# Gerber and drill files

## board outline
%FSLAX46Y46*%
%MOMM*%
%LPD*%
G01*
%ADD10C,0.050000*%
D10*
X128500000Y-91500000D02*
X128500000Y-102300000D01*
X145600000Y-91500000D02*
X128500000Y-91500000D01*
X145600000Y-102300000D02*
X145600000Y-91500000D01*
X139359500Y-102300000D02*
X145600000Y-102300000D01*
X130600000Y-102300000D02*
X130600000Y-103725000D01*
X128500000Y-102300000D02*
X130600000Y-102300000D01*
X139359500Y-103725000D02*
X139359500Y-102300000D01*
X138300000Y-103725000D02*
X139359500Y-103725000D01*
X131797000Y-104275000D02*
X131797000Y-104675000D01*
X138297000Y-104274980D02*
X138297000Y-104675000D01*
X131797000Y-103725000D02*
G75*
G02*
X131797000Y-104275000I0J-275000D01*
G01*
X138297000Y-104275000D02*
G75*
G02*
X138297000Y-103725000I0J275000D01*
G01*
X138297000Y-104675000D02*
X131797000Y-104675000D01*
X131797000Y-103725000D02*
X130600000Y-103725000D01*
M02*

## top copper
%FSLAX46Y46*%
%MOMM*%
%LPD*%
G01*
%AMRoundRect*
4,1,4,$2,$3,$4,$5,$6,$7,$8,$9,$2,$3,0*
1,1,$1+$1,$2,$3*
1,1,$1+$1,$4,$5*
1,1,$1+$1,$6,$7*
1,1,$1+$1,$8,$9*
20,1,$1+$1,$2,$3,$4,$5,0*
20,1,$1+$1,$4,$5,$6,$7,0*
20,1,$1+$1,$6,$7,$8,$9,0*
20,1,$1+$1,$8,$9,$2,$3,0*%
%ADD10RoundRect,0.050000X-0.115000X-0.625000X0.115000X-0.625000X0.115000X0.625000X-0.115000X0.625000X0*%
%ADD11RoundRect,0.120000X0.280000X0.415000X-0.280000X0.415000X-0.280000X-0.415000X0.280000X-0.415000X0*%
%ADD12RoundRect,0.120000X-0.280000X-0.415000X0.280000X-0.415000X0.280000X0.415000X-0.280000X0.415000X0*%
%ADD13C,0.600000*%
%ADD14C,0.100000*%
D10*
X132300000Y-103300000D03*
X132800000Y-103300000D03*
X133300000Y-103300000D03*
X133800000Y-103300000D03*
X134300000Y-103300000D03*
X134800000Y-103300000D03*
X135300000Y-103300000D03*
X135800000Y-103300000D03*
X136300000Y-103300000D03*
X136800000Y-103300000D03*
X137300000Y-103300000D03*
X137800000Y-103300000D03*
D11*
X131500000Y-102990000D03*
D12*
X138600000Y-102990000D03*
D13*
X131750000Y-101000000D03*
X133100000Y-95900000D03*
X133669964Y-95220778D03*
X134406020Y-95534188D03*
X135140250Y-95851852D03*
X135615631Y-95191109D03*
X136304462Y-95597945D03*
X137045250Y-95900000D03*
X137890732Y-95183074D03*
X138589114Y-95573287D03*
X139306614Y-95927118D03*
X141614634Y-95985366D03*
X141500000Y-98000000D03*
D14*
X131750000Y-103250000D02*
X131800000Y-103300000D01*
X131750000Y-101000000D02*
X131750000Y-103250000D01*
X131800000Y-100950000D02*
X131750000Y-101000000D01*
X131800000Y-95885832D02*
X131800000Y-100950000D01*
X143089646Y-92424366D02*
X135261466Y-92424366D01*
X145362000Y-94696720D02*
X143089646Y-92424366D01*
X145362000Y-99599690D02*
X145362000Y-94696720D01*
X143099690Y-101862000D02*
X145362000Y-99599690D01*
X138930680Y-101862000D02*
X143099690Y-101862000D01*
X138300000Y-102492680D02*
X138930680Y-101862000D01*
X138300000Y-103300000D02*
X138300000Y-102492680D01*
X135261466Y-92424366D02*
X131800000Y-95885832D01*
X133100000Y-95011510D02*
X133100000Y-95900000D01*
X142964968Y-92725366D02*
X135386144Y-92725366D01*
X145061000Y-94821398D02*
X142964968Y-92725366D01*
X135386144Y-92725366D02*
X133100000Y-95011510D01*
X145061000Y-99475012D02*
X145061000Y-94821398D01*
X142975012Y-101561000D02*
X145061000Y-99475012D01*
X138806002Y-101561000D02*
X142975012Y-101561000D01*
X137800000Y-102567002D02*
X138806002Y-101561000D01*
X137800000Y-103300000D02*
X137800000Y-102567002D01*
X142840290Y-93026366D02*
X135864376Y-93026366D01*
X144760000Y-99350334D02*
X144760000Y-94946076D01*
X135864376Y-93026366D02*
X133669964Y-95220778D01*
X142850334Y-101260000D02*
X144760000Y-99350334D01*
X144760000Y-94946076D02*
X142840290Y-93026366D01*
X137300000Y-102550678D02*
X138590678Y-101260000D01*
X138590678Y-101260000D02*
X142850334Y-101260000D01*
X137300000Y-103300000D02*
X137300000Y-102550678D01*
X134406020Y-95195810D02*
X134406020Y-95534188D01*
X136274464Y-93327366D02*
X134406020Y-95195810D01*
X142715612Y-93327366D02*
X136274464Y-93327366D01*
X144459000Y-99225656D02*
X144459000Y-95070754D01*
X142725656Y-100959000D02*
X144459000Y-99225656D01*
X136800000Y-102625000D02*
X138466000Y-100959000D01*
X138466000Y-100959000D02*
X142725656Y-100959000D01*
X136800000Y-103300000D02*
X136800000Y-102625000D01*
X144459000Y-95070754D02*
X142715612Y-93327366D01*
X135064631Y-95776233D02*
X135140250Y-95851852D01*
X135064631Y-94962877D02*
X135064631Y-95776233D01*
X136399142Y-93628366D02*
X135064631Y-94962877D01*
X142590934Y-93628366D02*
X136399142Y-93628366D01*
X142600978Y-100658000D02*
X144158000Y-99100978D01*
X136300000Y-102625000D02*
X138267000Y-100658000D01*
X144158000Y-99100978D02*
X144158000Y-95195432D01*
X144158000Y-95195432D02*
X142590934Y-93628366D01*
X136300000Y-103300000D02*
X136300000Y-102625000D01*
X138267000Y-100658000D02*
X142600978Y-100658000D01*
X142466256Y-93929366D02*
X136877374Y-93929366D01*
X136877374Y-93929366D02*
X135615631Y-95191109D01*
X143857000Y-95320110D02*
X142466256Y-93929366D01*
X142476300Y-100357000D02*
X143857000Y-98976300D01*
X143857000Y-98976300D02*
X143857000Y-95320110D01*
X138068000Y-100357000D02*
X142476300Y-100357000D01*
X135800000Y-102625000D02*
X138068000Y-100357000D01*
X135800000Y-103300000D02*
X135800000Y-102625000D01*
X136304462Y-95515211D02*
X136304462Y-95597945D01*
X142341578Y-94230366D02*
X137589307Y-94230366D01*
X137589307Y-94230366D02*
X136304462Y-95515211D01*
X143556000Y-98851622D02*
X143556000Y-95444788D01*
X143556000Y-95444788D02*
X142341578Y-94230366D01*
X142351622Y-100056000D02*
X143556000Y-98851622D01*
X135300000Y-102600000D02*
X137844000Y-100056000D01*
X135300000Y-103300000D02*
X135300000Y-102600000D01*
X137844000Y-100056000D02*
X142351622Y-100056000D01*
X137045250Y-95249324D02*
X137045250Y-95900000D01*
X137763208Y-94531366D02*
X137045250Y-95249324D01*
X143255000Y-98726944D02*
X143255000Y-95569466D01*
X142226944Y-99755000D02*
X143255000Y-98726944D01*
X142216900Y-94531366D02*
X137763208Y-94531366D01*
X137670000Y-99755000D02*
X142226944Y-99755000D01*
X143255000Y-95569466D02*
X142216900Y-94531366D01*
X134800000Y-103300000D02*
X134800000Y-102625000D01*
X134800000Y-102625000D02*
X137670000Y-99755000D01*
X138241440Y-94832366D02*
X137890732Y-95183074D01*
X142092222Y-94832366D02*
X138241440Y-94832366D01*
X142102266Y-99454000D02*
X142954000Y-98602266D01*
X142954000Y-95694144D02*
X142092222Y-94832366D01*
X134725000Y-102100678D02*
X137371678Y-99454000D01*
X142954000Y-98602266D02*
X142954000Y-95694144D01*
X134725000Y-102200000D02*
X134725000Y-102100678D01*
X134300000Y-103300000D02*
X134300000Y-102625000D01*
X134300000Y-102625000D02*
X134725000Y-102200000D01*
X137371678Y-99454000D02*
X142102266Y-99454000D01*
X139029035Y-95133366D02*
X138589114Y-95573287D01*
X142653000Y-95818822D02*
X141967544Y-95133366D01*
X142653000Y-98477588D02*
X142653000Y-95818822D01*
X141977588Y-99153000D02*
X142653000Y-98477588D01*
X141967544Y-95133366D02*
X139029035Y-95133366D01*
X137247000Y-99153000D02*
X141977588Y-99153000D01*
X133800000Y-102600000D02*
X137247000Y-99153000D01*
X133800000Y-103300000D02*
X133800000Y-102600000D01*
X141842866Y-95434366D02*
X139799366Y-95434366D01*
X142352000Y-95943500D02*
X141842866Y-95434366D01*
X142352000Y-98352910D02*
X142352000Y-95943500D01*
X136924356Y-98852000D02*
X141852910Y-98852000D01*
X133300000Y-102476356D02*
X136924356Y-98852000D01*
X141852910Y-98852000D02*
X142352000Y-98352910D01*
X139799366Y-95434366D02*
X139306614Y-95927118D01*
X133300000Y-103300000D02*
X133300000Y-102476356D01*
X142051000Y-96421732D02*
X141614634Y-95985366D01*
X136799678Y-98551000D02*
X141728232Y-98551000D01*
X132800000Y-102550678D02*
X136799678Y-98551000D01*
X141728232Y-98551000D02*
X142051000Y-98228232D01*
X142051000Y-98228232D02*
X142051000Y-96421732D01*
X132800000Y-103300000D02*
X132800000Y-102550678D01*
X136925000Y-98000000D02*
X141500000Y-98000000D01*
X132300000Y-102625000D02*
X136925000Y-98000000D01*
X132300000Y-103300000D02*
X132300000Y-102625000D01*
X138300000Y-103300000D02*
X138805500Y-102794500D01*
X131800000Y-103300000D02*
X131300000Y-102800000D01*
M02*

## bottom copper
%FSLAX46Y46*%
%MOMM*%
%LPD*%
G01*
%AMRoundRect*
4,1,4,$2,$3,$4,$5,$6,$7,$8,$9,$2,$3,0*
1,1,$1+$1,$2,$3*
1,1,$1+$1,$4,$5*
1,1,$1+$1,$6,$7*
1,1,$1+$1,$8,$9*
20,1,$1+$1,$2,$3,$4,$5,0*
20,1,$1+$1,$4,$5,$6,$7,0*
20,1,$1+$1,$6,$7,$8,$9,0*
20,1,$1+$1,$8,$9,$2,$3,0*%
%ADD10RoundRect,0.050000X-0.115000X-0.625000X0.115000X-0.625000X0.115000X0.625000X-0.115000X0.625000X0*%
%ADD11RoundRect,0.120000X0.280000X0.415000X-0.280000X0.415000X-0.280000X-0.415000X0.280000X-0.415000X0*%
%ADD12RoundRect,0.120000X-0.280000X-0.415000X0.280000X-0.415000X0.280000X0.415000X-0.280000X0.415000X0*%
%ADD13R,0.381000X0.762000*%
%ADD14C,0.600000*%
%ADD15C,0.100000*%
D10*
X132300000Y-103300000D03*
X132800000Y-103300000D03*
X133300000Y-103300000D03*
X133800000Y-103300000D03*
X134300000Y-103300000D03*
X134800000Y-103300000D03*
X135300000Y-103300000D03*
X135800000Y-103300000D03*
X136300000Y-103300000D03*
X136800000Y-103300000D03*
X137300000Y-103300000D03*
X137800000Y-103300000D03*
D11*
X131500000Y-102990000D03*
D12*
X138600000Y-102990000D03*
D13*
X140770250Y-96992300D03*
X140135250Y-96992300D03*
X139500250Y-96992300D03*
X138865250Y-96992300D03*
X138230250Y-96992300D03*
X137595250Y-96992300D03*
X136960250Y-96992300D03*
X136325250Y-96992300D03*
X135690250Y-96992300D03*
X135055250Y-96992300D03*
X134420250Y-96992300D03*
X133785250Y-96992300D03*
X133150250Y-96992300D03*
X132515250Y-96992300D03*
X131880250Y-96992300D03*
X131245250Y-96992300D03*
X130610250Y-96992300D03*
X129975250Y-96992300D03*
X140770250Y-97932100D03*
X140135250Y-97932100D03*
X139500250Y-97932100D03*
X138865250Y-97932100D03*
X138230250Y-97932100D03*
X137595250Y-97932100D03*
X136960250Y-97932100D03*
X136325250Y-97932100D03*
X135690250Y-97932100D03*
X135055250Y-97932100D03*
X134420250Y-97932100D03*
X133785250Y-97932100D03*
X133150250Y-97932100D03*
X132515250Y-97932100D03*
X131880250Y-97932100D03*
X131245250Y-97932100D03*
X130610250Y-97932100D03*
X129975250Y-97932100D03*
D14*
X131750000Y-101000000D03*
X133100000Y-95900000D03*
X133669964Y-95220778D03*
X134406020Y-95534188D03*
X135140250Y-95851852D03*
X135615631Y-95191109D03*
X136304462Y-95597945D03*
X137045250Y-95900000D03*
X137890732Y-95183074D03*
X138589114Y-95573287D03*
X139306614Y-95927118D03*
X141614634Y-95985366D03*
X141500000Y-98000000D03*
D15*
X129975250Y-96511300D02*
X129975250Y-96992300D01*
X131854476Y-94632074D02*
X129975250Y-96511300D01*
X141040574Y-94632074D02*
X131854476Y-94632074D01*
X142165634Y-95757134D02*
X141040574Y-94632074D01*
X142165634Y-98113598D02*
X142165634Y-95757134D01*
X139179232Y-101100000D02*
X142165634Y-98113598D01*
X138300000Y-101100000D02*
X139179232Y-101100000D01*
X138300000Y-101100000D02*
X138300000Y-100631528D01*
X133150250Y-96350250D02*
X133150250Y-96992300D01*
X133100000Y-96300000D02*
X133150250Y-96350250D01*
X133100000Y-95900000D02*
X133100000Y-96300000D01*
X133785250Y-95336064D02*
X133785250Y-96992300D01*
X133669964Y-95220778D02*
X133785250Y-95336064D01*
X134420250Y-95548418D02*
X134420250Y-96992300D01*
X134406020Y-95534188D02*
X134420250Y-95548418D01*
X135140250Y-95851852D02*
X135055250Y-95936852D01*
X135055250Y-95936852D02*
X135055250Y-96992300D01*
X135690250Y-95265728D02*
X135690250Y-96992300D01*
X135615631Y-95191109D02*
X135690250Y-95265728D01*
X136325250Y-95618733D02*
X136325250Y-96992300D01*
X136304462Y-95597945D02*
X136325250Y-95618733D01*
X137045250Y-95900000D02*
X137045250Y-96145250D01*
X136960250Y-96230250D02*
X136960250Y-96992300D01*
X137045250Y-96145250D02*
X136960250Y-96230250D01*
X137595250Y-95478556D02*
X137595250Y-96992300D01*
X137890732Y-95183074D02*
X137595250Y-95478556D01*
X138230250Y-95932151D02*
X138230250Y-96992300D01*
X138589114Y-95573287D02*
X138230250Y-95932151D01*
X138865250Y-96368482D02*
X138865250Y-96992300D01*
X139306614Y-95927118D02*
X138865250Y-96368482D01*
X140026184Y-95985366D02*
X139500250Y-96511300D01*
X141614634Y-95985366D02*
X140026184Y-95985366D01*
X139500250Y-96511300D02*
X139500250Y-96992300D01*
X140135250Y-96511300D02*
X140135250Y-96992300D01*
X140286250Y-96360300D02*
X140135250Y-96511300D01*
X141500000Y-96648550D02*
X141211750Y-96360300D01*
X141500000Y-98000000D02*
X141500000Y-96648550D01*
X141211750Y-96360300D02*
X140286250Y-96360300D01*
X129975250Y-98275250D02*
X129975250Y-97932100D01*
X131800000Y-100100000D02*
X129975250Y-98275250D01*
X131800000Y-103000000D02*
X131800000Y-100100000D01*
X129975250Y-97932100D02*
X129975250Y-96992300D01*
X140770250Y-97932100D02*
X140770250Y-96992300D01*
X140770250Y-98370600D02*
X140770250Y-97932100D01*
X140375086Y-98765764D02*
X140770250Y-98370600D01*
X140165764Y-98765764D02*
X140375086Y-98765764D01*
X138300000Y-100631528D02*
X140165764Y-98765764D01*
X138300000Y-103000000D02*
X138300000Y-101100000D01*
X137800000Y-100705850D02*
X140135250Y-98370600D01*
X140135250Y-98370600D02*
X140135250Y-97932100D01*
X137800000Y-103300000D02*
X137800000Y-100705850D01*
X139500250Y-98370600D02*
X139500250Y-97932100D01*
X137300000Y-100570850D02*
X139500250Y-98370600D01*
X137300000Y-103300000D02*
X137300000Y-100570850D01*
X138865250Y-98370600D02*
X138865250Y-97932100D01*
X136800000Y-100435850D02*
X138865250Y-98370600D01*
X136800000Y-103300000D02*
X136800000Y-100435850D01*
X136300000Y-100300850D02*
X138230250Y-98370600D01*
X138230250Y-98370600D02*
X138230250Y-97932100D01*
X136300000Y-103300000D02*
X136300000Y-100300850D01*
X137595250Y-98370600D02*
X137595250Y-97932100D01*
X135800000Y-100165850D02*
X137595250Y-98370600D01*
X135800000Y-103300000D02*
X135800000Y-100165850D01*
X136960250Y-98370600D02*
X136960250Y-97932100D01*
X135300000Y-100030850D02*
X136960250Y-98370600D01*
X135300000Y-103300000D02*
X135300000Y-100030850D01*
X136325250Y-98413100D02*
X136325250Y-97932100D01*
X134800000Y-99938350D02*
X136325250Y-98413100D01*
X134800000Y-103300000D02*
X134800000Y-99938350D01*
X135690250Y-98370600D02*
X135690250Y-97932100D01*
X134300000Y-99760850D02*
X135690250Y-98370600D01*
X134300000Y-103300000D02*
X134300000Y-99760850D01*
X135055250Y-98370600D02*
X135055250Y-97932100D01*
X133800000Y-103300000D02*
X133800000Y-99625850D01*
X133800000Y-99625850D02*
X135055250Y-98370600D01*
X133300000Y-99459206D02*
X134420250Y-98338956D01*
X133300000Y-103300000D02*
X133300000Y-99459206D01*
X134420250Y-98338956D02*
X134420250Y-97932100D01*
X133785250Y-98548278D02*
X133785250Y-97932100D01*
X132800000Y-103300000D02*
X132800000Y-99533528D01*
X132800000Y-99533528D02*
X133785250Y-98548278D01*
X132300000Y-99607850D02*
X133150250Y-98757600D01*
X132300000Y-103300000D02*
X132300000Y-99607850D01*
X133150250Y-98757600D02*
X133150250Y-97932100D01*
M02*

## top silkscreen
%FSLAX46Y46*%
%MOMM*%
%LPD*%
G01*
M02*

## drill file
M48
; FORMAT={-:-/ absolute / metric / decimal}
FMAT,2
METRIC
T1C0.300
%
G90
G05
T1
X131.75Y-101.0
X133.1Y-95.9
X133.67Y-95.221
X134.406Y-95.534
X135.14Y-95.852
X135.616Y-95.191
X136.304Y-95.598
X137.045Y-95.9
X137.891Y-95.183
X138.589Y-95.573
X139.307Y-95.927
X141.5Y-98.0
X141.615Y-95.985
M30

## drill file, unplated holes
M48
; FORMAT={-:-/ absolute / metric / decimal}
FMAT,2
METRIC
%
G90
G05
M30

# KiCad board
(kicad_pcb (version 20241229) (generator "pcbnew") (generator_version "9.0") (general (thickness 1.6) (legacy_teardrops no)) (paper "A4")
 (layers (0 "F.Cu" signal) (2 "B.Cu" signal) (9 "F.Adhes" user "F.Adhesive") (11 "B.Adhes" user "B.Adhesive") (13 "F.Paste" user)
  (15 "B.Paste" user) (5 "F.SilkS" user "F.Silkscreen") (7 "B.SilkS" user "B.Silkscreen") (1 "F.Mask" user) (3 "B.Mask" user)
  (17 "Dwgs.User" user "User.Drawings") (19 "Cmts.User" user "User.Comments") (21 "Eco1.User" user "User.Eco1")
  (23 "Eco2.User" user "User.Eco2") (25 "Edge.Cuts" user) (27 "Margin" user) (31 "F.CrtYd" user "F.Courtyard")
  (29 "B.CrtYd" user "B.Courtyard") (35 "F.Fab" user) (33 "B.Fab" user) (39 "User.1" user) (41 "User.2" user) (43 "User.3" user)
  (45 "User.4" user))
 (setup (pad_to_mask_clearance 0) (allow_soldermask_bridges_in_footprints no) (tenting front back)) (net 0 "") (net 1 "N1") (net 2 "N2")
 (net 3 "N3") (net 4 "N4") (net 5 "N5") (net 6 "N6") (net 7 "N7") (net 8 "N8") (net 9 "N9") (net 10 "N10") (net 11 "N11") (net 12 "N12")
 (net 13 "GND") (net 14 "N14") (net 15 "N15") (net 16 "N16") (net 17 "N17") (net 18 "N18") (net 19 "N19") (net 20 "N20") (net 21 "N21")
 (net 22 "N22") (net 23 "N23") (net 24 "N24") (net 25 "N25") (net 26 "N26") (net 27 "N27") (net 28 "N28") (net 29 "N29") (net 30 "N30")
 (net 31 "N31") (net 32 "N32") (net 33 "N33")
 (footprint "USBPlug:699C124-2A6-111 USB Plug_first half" (layer "F.Cu") (at 134.8 100.3)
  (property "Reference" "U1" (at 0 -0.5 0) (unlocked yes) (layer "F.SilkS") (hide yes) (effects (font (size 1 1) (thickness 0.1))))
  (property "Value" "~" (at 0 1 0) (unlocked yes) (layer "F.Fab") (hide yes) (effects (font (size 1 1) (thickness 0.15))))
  (pad "0" smd roundrect (at -2.5 3) (size 0.33 1.35) (layers "F.Cu" "F.Mask" "F.Paste") (roundrect_rratio 0.1515151515) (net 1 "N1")
   (thermal_bridge_angle 45))
  (pad "1" smd roundrect (at -2 3) (size 0.33 1.35) (layers "F.Cu" "F.Mask" "F.Paste") (roundrect_rratio 0.1515151515) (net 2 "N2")
   (thermal_bridge_angle 45))
  (pad "2" smd roundrect (at -1.5 3) (size 0.33 1.35) (layers "F.Cu" "F.Mask" "F.Paste") (roundrect_rratio 0.1515151515) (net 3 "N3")
   (thermal_bridge_angle 45))
  (pad "3" smd roundrect (at -1 3) (size 0.33 1.35) (layers "F.Cu" "F.Mask" "F.Paste") (roundrect_rratio 0.1515151515) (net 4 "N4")
   (thermal_bridge_angle 45))
  (pad "4" smd roundrect (at -0.5 3) (size 0.33 1.35) (layers "F.Cu" "F.Mask" "F.Paste") (roundrect_rratio 0.1515151515) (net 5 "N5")
   (thermal_bridge_angle 45))
  (pad "5" smd roundrect (at 0 3) (size 0.33 1.35) (layers "F.Cu" "F.Mask" "F.Paste") (roundrect_rratio 0.1515151515) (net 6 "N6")
   (thermal_bridge_angle 45))
  (pad "6" smd roundrect (at 0.5 3) (size 0.33 1.35) (layers "F.Cu" "F.Mask" "F.Paste") (roundrect_rratio 0.1515151515) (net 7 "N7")
   (thermal_bridge_angle 45))
  (pad "7" smd roundrect (at 1 3) (size 0.33 1.35) (layers "F.Cu" "F.Mask" "F.Paste") (roundrect_rratio 0.1515151515) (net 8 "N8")
   (thermal_bridge_angle 45))
  (pad "8" smd roundrect (at 1.5 3) (size 0.33 1.35) (layers "F.Cu" "F.Mask" "F.Paste") (roundrect_rratio 0.1515151515) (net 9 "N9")
   (thermal_bridge_angle 45))
  (pad "9" smd roundrect (at 2 3) (size 0.33 1.35) (layers "F.Cu" "F.Mask" "F.Paste") (roundrect_rratio 0.1515151515) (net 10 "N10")
   (thermal_bridge_angle 45))
  (pad "10" smd roundrect (at 2.5 3) (size 0.33 1.35) (layers "F.Cu" "F.Mask" "F.Paste") (roundrect_rratio 0.1515151515) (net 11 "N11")
   (thermal_bridge_angle 45))
  (pad "11" smd roundrect (at 3 3) (size 0.33 1.35) (layers "F.Cu" "F.Mask" "F.Paste") (roundrect_rratio 0.1515151515) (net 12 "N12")
   (thermal_bridge_angle 45))
  (pad "24" smd roundrect (at -3 3 180) (size 0.8 1.07) (drill (offset 0.3 0.31)) (layers "F.Cu" "F.Mask" "F.Paste") (roundrect_rratio 0.15)
   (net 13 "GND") (thermal_bridge_angle 45))
  (pad "25" smd roundrect (at 3.5 3) (size 0.8 1.07) (drill (offset 0.3 -0.31)) (layers "F.Cu" "F.Mask" "F.Paste") (roundrect_rratio 0.15)
   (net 13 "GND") (thermal_bridge_angle 45)))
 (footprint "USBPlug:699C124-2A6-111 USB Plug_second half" (layer "B.Cu") (at 134.8 106.3)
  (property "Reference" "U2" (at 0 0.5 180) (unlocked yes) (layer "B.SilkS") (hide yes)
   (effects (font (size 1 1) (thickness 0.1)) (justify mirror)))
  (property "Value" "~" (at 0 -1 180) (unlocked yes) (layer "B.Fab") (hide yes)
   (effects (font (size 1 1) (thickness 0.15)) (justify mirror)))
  (pad "12" smd roundrect (at -2.5 -3) (size 0.33 1.35) (layers "B.Cu" "B.Mask" "B.Paste") (roundrect_rratio 0.1515151515) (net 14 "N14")
   (thermal_bridge_angle 45))
  (pad "13" smd roundrect (at -2 -3) (size 0.33 1.35) (layers "B.Cu" "B.Mask" "B.Paste") (roundrect_rratio 0.1515151515) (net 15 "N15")
   (thermal_bridge_angle 45))
  (pad "14" smd roundrect (at -1.5 -3) (size 0.33 1.35) (layers "B.Cu" "B.Mask" "B.Paste") (roundrect_rratio 0.1515151515) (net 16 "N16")
   (thermal_bridge_angle 45))
  (pad "15" smd roundrect (at -1 -3) (size 0.33 1.35) (layers "B.Cu" "B.Mask" "B.Paste") (roundrect_rratio 0.1515151515) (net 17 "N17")
   (thermal_bridge_angle 45))
  (pad "16" smd roundrect (at -0.5 -3) (size 0.33 1.35) (layers "B.Cu" "B.Mask" "B.Paste") (roundrect_rratio 0.1515151515) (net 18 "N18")
   (thermal_bridge_angle 45))
  (pad "17" smd roundrect (at 0 -3) (size 0.33 1.35) (layers "B.Cu" "B.Mask" "B.Paste") (roundrect_rratio 0.1515151515) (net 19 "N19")
   (thermal_bridge_angle 45))
  (pad "18" smd roundrect (at 0.5 -3) (size 0.33 1.35) (layers "B.Cu" "B.Mask" "B.Paste") (roundrect_rratio 0.1515151515) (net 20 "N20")
   (thermal_bridge_angle 45))
  (pad "19" smd roundrect (at 1 -3) (size 0.33 1.35) (layers "B.Cu" "B.Mask" "B.Paste") (roundrect_rratio 0.1515151515) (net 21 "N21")
   (thermal_bridge_angle 45))
  (pad "20" smd roundrect (at 1.5 -3) (size 0.33 1.35) (layers "B.Cu" "B.Mask" "B.Paste") (roundrect_rratio 0.1515151515) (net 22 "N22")
   (thermal_bridge_angle 45))
  (pad "21" smd roundrect (at 2 -3) (size 0.33 1.35) (layers "B.Cu" "B.Mask" "B.Paste") (roundrect_rratio 0.1515151515) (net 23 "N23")
   (thermal_bridge_angle 45))
  (pad "22" smd roundrect (at 2.5 -3) (size 0.33 1.35) (layers "B.Cu" "B.Mask" "B.Paste") (roundrect_rratio 0.1515151515) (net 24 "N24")
   (thermal_bridge_angle 45))
  (pad "23" smd roundrect (at 3 -3) (size 0.33 1.35) (layers "B.Cu" "B.Mask" "B.Paste") (roundrect_rratio 0.1515151515) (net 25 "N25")
   (thermal_bridge_angle 45))
  (pad "26" smd roundrect (at -3 -3.3 180) (size 0.8 1.07) (drill (offset 0.3 0.01)) (layers "B.Cu" "B.Mask" "B.Paste")
   (roundrect_rratio 0.15) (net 13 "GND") (thermal_bridge_angle 45))
  (pad "27" smd roundrect (at 3.5 -3.3) (size 0.8 1.07) (drill (offset 0.3 -0.01)) (layers "B.Cu" "B.Mask" "B.Paste")
   (roundrect_rratio 0.15) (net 13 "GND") (thermal_bridge_angle 45)))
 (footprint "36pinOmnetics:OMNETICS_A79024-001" (layer "B.Cu") (at 135.37275 97.4622)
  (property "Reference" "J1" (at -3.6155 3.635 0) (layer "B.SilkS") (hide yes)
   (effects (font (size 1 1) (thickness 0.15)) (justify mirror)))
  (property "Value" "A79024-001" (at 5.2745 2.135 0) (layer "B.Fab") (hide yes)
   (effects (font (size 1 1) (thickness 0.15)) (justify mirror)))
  (pad "1" smd rect (at 5.3975 -0.4699) (size 0.381 0.762) (layers "B.Cu" "B.Mask" "B.Paste") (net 13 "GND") (solder_mask_margin 0.102))
  (pad "2" smd rect (at 4.7625 -0.4699) (size 0.381 0.762) (layers "B.Cu" "B.Mask" "B.Paste") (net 1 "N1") (solder_mask_margin 0.102))
  (pad "3" smd rect (at 4.1275 -0.4699) (size 0.381 0.762) (layers "B.Cu" "B.Mask" "B.Paste") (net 2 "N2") (solder_mask_margin 0.102))
  (pad "4" smd rect (at 3.4925 -0.4699) (size 0.381 0.762) (layers "B.Cu" "B.Mask" "B.Paste") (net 3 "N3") (solder_mask_margin 0.102))
  (pad "5" smd rect (at 2.8575 -0.4699) (size 0.381 0.762) (layers "B.Cu" "B.Mask" "B.Paste") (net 4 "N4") (solder_mask_margin 0.102))
  (pad "6" smd rect (at 2.2225 -0.4699) (size 0.381 0.762) (layers "B.Cu" "B.Mask" "B.Paste") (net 5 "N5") (solder_mask_margin 0.102))
  (pad "7" smd rect (at 1.5875 -0.4699) (size 0.381 0.762) (layers "B.Cu" "B.Mask" "B.Paste") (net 6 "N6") (solder_mask_margin 0.102))
  (pad "8" smd rect (at 0.9525 -0.4699) (size 0.381 0.762) (layers "B.Cu" "B.Mask" "B.Paste") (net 7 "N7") (solder_mask_margin 0.102))
  (pad "9" smd rect (at 0.3175 -0.4699) (size 0.381 0.762) (layers "B.Cu" "B.Mask" "B.Paste") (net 8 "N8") (solder_mask_margin 0.102))
  (pad "10" smd rect (at -0.3175 -0.4699) (size 0.381 0.762) (layers "B.Cu" "B.Mask" "B.Paste") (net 9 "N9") (solder_mask_margin 0.102))
  (pad "11" smd rect (at -0.9525 -0.4699) (size 0.381 0.762) (layers "B.Cu" "B.Mask" "B.Paste") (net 10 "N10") (solder_mask_margin 0.102))
  (pad "12" smd rect (at -1.5875 -0.4699) (size 0.381 0.762) (layers "B.Cu" "B.Mask" "B.Paste") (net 11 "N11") (solder_mask_margin 0.102))
  (pad "13" smd rect (at -2.2225 -0.4699) (size 0.381 0.762) (layers "B.Cu" "B.Mask" "B.Paste") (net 12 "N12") (solder_mask_margin 0.102))
  (pad "14" smd rect (at -2.8575 -0.4699) (size 0.381 0.762) (layers "B.Cu" "B.Mask" "B.Paste") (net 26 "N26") (solder_mask_margin 0.102))
  (pad "15" smd rect (at -3.4925 -0.4699) (size 0.381 0.762) (layers "B.Cu" "B.Mask" "B.Paste") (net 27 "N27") (solder_mask_margin 0.102))
  (pad "16" smd rect (at -4.1275 -0.4699) (size 0.381 0.762) (layers "B.Cu" "B.Mask" "B.Paste") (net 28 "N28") (solder_mask_margin 0.102))
  (pad "17" smd rect (at -4.7625 -0.4699) (size 0.381 0.762) (layers "B.Cu" "B.Mask" "B.Paste") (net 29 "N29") (solder_mask_margin 0.102))
  (pad "18" smd rect (at -5.3975 -0.4699) (size 0.381 0.762) (layers "B.Cu" "B.Mask" "B.Paste") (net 13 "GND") (solder_mask_margin 0.102))
  (pad "19" smd rect (at 5.3975 0.4699) (size 0.381 0.762) (layers "B.Cu" "B.Mask" "B.Paste") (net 13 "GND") (solder_mask_margin 0.102))
  (pad "20" smd rect (at 4.7625 0.4699) (size 0.381 0.762) (layers "B.Cu" "B.Mask" "B.Paste") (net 25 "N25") (solder_mask_margin 0.102))
  (pad "21" smd rect (at 4.1275 0.4699) (size 0.381 0.762) (layers "B.Cu" "B.Mask" "B.Paste") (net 24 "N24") (solder_mask_margin 0.102))
  (pad "22" smd rect (at 3.4925 0.4699) (size 0.381 0.762) (layers "B.Cu" "B.Mask" "B.Paste") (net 23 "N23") (solder_mask_margin 0.102))
  (pad "23" smd rect (at 2.8575 0.4699) (size 0.381 0.762) (layers "B.Cu" "B.Mask" "B.Paste") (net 22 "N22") (solder_mask_margin 0.102))
  (pad "24" smd rect (at 2.2225 0.4699) (size 0.381 0.762) (layers "B.Cu" "B.Mask" "B.Paste") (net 21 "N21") (solder_mask_margin 0.102))
  (pad "25" smd rect (at 1.5875 0.4699) (size 0.381 0.762) (layers "B.Cu" "B.Mask" "B.Paste") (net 20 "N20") (solder_mask_margin 0.102))
  (pad "26" smd rect (at 0.9525 0.4699) (size 0.381 0.762) (layers "B.Cu" "B.Mask" "B.Paste") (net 19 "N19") (solder_mask_margin 0.102))
  (pad "27" smd rect (at 0.3175 0.4699) (size 0.381 0.762) (layers "B.Cu" "B.Mask" "B.Paste") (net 18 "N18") (solder_mask_margin 0.102))
  (pad "28" smd rect (at -0.3175 0.4699) (size 0.381 0.762) (layers "B.Cu" "B.Mask" "B.Paste") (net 17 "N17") (solder_mask_margin 0.102))
  (pad "29" smd rect (at -0.9525 0.4699) (size 0.381 0.762) (layers "B.Cu" "B.Mask" "B.Paste") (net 16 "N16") (solder_mask_margin 0.102))
  (pad "30" smd rect (at -1.5875 0.4699) (size 0.381 0.762) (layers "B.Cu" "B.Mask" "B.Paste") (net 15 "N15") (solder_mask_margin 0.102))
  (pad "31" smd rect (at -2.2225 0.4699) (size 0.381 0.762) (layers "B.Cu" "B.Mask" "B.Paste") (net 14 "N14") (solder_mask_margin 0.102))
  (pad "32" smd rect (at -2.8575 0.4699) (size 0.381 0.762) (layers "B.Cu" "B.Mask" "B.Paste") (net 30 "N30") (solder_mask_margin 0.102))
  (pad "33" smd rect (at -3.4925 0.4699) (size 0.381 0.762) (layers "B.Cu" "B.Mask" "B.Paste") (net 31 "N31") (solder_mask_margin 0.102))
  (pad "34" smd rect (at -4.1275 0.4699) (size 0.381 0.762) (layers "B.Cu" "B.Mask" "B.Paste") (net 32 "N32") (solder_mask_margin 0.102))
  (pad "35" smd rect (at -4.7625 0.4699) (size 0.381 0.762) (layers "B.Cu" "B.Mask" "B.Paste") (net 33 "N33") (solder_mask_margin 0.102))
  (pad "36" smd rect (at -5.3975 0.4699) (size 0.381 0.762) (layers "B.Cu" "B.Mask" "B.Paste") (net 13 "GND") (solder_mask_margin 0.102)))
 (gr_line (start 139.3595 102.3) (end 145.6 102.3) (stroke (width 0.05) (type default)) (layer "Edge.Cuts"))
 (gr_line (start 145.6 102.3) (end 145.6 91.5) (stroke (width 0.05) (type default)) (layer "Edge.Cuts"))
 (gr_line (start 145.6 91.5) (end 128.5 91.5) (stroke (width 0.05) (type default)) (layer "Edge.Cuts"))
 (gr_line (start 138.3 103.725) (end 139.3595 103.725) (stroke (width 0.05) (type default)) (layer "Edge.Cuts"))
 (gr_line (start 131.797 104.275) (end 131.797 104.675) (stroke (width 0.05) (type default)) (layer "Edge.Cuts"))
 (gr_line (start 130.6 102.3) (end 130.6 103.725) (stroke (width 0.05) (type default)) (layer "Edge.Cuts"))
 (gr_line (start 138.297 104.27498) (end 138.297 104.675) (stroke (width 0.05) (type default)) (layer "Edge.Cuts"))
 (gr_arc (start 131.797 103.725) (mid 132.072 104) (end 131.797 104.275) (stroke (width 0.05) (type default)) (layer "Edge.Cuts"))
 (gr_arc (start 138.297 104.275) (mid 138.022 104) (end 138.297 103.725) (stroke (width 0.05) (type default)) (layer "Edge.Cuts"))
 (gr_line (start 128.5 102.3) (end 130.6 102.3) (stroke (width 0.05) (type default)) (layer "Edge.Cuts"))
 (gr_line (start 138.297 104.675) (end 131.797 104.675) (stroke (width 0.05) (type default)) (layer "Edge.Cuts"))
 (gr_line (start 139.3595 103.725) (end 139.3595 102.3) (stroke (width 0.05) (type default)) (layer "Edge.Cuts"))
 (gr_line (start 128.5 91.5) (end 128.5 102.3) (stroke (width 0.05) (type default)) (layer "Edge.Cuts"))
 (gr_line (start 131.797 103.725) (end 130.6 103.725) (stroke (width 0.05) (type default)) (layer "Edge.Cuts"))
 (segment (start 145.362 94.69672) (end 143.089646 92.424366) (width 0.1) (layer "F.Cu") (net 13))
 (segment (start 138.3 103.3) (end 138.8055 102.7945) (width 0.1) (layer "F.Cu") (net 13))
 (segment (start 131.8 100.95) (end 131.75 101) (width 0.1) (layer "F.Cu") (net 13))
 (segment (start 143.089646 92.424366) (end 135.261466 92.424366) (width 0.1) (layer "F.Cu") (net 13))
 (segment (start 131.75 101) (end 131.75 103.25) (width 0.1) (layer "F.Cu") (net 13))
 (segment (start 138.93068 101.862) (end 143.09969 101.862) (width 0.1) (layer "F.Cu") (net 13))
 (segment (start 145.362 99.59969) (end 145.362 94.69672) (width 0.1) (layer "F.Cu") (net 13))
 (segment (start 131.8 95.885832) (end 131.8 100.95) (width 0.1) (layer "F.Cu") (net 13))
 (segment (start 131.75 103.25) (end 131.8 103.3) (width 0.1) (layer "F.Cu") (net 13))
 (segment (start 135.261466 92.424366) (end 131.8 95.885832) (width 0.1) (layer "F.Cu") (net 13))
 (segment (start 138.3 103.3) (end 138.3 102.49268) (width 0.1) (layer "F.Cu") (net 13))
 (segment (start 143.09969 101.862) (end 145.362 99.59969) (width 0.1) (layer "F.Cu") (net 13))
 (segment (start 131.8 103.3) (end 131.3 102.8) (width 0.1) (layer "F.Cu") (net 13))
 (segment (start 138.3 102.49268) (end 138.93068 101.862) (width 0.1) (layer "F.Cu") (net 13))
 (via (at 131.75 101) (size 0.6) (drill 0.3) (layers "F.Cu" "B.Cu") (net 13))
 (segment (start 131.854476 94.632074) (end 129.97525 96.5113) (width 0.1) (layer "B.Cu") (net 13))
 (segment (start 139.179232 101.1) (end 142.165634 98.113598) (width 0.1) (layer "B.Cu") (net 13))
 (segment (start 138.3 100.631528) (end 140.165764 98.765764) (width 0.1) (layer "B.Cu") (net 13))
 (segment (start 141.040574 94.632074) (end 131.854476 94.632074) (width 0.1) (layer "B.Cu") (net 13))
 (segment (start 129.97525 97.9321) (end 129.97525 96.9923) (width 0.1) (layer "B.Cu") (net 13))
 (segment (start 131.8 100.1) (end 129.97525 98.27525) (width 0.1) (layer "B.Cu") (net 13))
 (segment (start 138.3 101.1) (end 139.179232 101.1) (width 0.1) (layer "B.Cu") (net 13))
 (segment (start 142.165634 98.113598) (end 142.165634 95.757134) (width 0.1) (layer "B.Cu") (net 13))
 (segment (start 140.165764 98.765764) (end 140.375086 98.765764) (width 0.1) (layer "B.Cu") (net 13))
 (segment (start 142.165634 95.757134) (end 141.040574 94.632074) (width 0.1) (layer "B.Cu") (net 13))
 (segment (start 140.77025 97.9321) (end 140.77025 96.9923) (width 0.1) (layer "B.Cu") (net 13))
 (segment (start 129.97525 96.5113) (end 129.97525 96.9923) (width 0.1) (layer "B.Cu") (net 13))
 (segment (start 140.375086 98.765764) (end 140.77025 98.3706) (width 0.1) (layer "B.Cu") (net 13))
 (segment (start 129.97525 98.27525) (end 129.97525 97.9321) (width 0.1) (layer "B.Cu") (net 13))
 (segment (start 131.8 103) (end 131.8 100.1) (width 0.1) (layer "B.Cu") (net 13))
 (segment (start 138.3 103) (end 138.3 101.1) (width 0.1) (layer "B.Cu") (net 13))
 (segment (start 138.3 101.1) (end 138.3 100.631528) (width 0.1) (layer "B.Cu") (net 13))
 (segment (start 140.77025 98.3706) (end 140.77025 97.9321) (width 0.1) (layer "B.Cu") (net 13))
 (segment (start 133.3 103.3) (end 133.3 102.476356) (width 0.1) (layer "F.Cu") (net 3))
 (segment (start 141.85291 98.852) (end 142.352 98.35291) (width 0.1) (layer "F.Cu") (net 3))
 (segment (start 139.799366 95.434366) (end 139.306614 95.927118) (width 0.1) (layer "F.Cu") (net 3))
 (segment (start 142.352 95.9435) (end 141.842866 95.434366) (width 0.1) (layer "F.Cu") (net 3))
 (segment (start 133.3 102.476356) (end 136.924356 98.852) (width 0.1) (layer "F.Cu") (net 3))
 (segment (start 142.352 98.35291) (end 142.352 95.9435) (width 0.1) (layer "F.Cu") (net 3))
 (segment (start 141.842866 95.434366) (end 139.799366 95.434366) (width 0.1) (layer "F.Cu") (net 3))
 (segment (start 136.924356 98.852) (end 141.85291 98.852) (width 0.1) (layer "F.Cu") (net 3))
 (via (at 139.306614 95.927118) (size 0.6) (drill 0.3) (layers "F.Cu" "B.Cu") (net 3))
 (segment (start 138.86525 96.368482) (end 138.86525 96.9923) (width 0.1) (layer "B.Cu") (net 3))
 (segment (start 139.306614 95.927118) (end 138.86525 96.368482) (width 0.1) (layer "B.Cu") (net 3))
 (segment (start 144.459 95.070754) (end 142.715612 93.327366) (width 0.1) (layer "F.Cu") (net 10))
 (segment (start 136.8 102.625) (end 138.466 100.959) (width 0.1) (layer "F.Cu") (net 10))
 (segment (start 142.725656 100.959) (end 144.459 99.225656) (width 0.1) (layer "F.Cu") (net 10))
 (segment (start 136.8 103.3) (end 136.8 102.625) (width 0.1) (layer "F.Cu") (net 10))
 (segment (start 144.459 99.225656) (end 144.459 95.070754) (width 0.1) (layer "F.Cu") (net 10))
 (segment (start 142.715612 93.327366) (end 136.274464 93.327366) (width 0.1) (layer "F.Cu") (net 10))
 (segment (start 136.274464 93.327366) (end 134.40602 95.19581) (width 0.1) (layer "F.Cu") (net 10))
 (segment (start 134.40602 95.19581) (end 134.40602 95.534188) (width 0.1) (layer "F.Cu") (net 10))
 (segment (start 138.466 100.959) (end 142.725656 100.959) (width 0.1) (layer "F.Cu") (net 10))
 (via (at 134.40602 95.534188) (size 0.6) (drill 0.3) (layers "F.Cu" "B.Cu") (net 10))
 (segment (start 134.42025 95.548418) (end 134.42025 96.9923) (width 0.1) (layer "B.Cu") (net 10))
 (segment (start 134.40602 95.534188) (end 134.42025 95.548418) (width 0.1) (layer "B.Cu") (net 10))
 (segment (start 134.3 102.625) (end 134.725 102.2) (width 0.1) (layer "F.Cu") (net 5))
 (segment (start 134.725 102.100678) (end 137.371678 99.454) (width 0.1) (layer "F.Cu") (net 5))
 (segment (start 142.954 98.602266) (end 142.954 95.694144) (width 0.1) (layer "F.Cu") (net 5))
 (segment (start 137.371678 99.454) (end 142.102266 99.454) (width 0.1) (layer "F.Cu") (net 5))
 (segment (start 142.954 95.694144) (end 142.092222 94.832366) (width 0.1) (layer "F.Cu") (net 5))
 (segment (start 142.102266 99.454) (end 142.954 98.602266) (width 0.1) (layer "F.Cu") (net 5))
 (segment (start 134.3 103.3) (end 134.3 102.625) (width 0.1) (layer "F.Cu") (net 5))
 (segment (start 138.24144 94.832366) (end 137.890732 95.183074) (width 0.1) (layer "F.Cu") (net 5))
 (segment (start 134.725 102.2) (end 134.725 102.100678) (width 0.1) (layer "F.Cu") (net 5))
 (segment (start 142.092222 94.832366) (end 138.24144 94.832366) (width 0.1) (layer "F.Cu") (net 5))
 (via (at 137.890732 95.183074) (size 0.6) (drill 0.3) (layers "F.Cu" "B.Cu") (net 5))
 (segment (start 137.890732 95.183074) (end 137.59525 95.478556) (width 0.1) (layer "B.Cu") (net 5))
 (segment (start 137.59525 95.478556) (end 137.59525 96.9923) (width 0.1) (layer "B.Cu") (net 5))
 (segment (start 138.068 100.357) (end 142.4763 100.357) (width 0.1) (layer "F.Cu") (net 8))
 (segment (start 143.857 95.32011) (end 142.466256 93.929366) (width 0.1) (layer "F.Cu") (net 8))
 (segment (start 142.466256 93.929366) (end 136.877374 93.929366) (width 0.1) (layer "F.Cu") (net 8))
 (segment (start 136.877374 93.929366) (end 135.615631 95.191109) (width 0.1) (layer "F.Cu") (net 8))
 (segment (start 142.4763 100.357) (end 143.857 98.9763) (width 0.1) (layer "F.Cu") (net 8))
 (segment (start 135.8 102.625) (end 138.068 100.357) (width 0.1) (layer "F.Cu") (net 8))
 (segment (start 143.857 98.9763) (end 143.857 95.32011) (width 0.1) (layer "F.Cu") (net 8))
 (segment (start 135.8 103.3) (end 135.8 102.625) (width 0.1) (layer "F.Cu") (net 8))
 (via (at 135.615631 95.191109) (size 0.6) (drill 0.3) (layers "F.Cu" "B.Cu") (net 8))
 (segment (start 135.69025 95.265728) (end 135.69025 96.9923) (width 0.1) (layer "B.Cu") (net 8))
 (segment (start 135.615631 95.191109) (end 135.69025 95.265728) (width 0.1) (layer "B.Cu") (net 8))
 (segment (start 135.8 103.3) (end 135.8 100.16585) (width 0.1) (layer "B.Cu") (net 21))
 (segment (start 137.59525 98.3706) (end 137.59525 97.9321) (width 0.1) (layer "B.Cu") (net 21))
 (segment (start 135.8 100.16585) (end 137.59525 98.3706) (width 0.1) (layer "B.Cu") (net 21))
 (segment (start 136.3 103.3) (end 136.3 100.30085) (width 0.1) (layer "B.Cu") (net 22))
 (segment (start 136.3 100.30085) (end 138.23025 98.3706) (width 0.1) (layer "B.Cu") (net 22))
 (segment (start 138.23025 98.3706) (end 138.23025 97.9321) (width 0.1) (layer "B.Cu") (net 22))
 (segment (start 137.3 102.550678) (end 138.590678 101.26) (width 0.1) (layer "F.Cu") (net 11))
 (segment (start 142.84029 93.026366) (end 135.864376 93.026366) (width 0.1) (layer "F.Cu") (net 11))
 (segment (start 142.850334 101.26) (end 144.76 99.350334) (width 0.1) (layer "F.Cu") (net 11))
 (segment (start 138.590678 101.26) (end 142.850334 101.26) (width 0.1) (layer "F.Cu") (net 11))
 (segment (start 144.76 94.946076) (end 142.84029 93.026366) (width 0.1) (layer "F.Cu") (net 11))
 (segment (start 144.76 99.350334) (end 144.76 94.946076) (width 0.1) (layer "F.Cu") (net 11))
 (segment (start 137.3 103.3) (end 137.3 102.550678) (width 0.1) (layer "F.Cu") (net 11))
 (segment (start 135.864376 93.026366) (end 133.669964 95.220778) (width 0.1) (layer "F.Cu") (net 11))
 (via (at 133.669964 95.220778) (size 0.6) (drill 0.3) (layers "F.Cu" "B.Cu") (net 11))
 (segment (start 133.78525 95.336064) (end 133.78525 96.9923) (width 0.1) (layer "B.Cu") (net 11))
 (segment (start 133.669964 95.220778) (end 133.78525 95.336064) (width 0.1) (layer "B.Cu") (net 11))
 (segment (start 134.8 103.3) (end 134.8 102.625) (width 0.1) (layer "F.Cu") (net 6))
 (segment (start 137.763208 94.531366) (end 137.04525 95.249324) (width 0.1) (layer "F.Cu") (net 6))
 (segment (start 137.04525 95.249324) (end 137.04525 95.9) (width 0.1) (layer "F.Cu") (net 6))
 (segment (start 143.255 95.569466) (end 142.2169 94.531366) (width 0.1) (layer "F.Cu") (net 6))
 (segment (start 134.8 102.625) (end 137.67 99.755) (width 0.1) (layer "F.Cu") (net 6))
 (segment (start 143.255 98.726944) (end 143.255 95.569466) (width 0.1) (layer "F.Cu") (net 6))
 (segment (start 142.226944 99.755) (end 143.255 98.726944) (width 0.1) (layer "F.Cu") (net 6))
 (segment (start 137.67 99.755) (end 142.226944 99.755) (width 0.1) (layer "F.Cu") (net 6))
 (segment (start 142.2169 94.531366) (end 137.763208 94.531366) (width 0.1) (layer "F.Cu") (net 6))
 (via (at 137.04525 95.9) (size 0.6) (drill 0.3) (layers "F.Cu" "B.Cu") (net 6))
 (segment (start 136.96025 96.23025) (end 136.96025 96.9923) (width 0.1) (layer "B.Cu") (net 6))
 (segment (start 137.04525 96.14525) (end 136.96025 96.23025) (width 0.1) (layer "B.Cu") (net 6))
 (segment (start 137.04525 95.9) (end 137.04525 96.14525) (width 0.1) (layer "B.Cu") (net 6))
 (segment (start 138.267 100.658) (end 142.600978 100.658) (width 0.1) (layer "F.Cu") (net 9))
 (segment (start 136.3 102.625) (end 138.267 100.658) (width 0.1) (layer "F.Cu") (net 9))
 (segment (start 136.399142 93.628366) (end 135.064631 94.962877) (width 0.1) (layer "F.Cu") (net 9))
 (segment (start 144.158 95.195432) (end 142.590934 93.628366) (width 0.1) (layer "F.Cu") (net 9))
 (segment (start 142.590934 93.628366) (end 136.399142 93.628366) (width 0.1) (layer "F.Cu") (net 9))
 (segment (start 135.064631 95.776233) (end 135.14025 95.851852) (width 0.1) (layer "F.Cu") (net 9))
 (segment (start 136.3 103.3) (end 136.3 102.625) (width 0.1) (layer "F.Cu") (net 9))
 (segment (start 144.158 99.100978) (end 144.158 95.195432) (width 0.1) (layer "F.Cu") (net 9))
 (segment (start 135.064631 94.962877) (end 135.064631 95.776233) (width 0.1) (layer "F.Cu") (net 9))
 (segment (start 142.600978 100.658) (end 144.158 99.100978) (width 0.1) (layer "F.Cu") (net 9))
 (via (at 135.14025 95.851852) (size 0.6) (drill 0.3) (layers "F.Cu" "B.Cu") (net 9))
 (segment (start 135.05525 95.936852) (end 135.05525 96.9923) (width 0.1) (layer "B.Cu") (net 9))
 (segment (start 135.14025 95.851852) (end 135.05525 95.936852) (width 0.1) (layer "B.Cu") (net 9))
 (segment (start 142.051 98.228232) (end 142.051 96.421732) (width 0.1) (layer "F.Cu") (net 2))
 (segment (start 142.051 96.421732) (end 141.614634 95.985366) (width 0.1) (layer "F.Cu") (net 2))
 (segment (start 132.8 102.550678) (end 136.799678 98.551) (width 0.1) (layer "F.Cu") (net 2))
 (segment (start 141.728232 98.551) (end 142.051 98.228232) (width 0.1) (layer "F.Cu") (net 2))
 (segment (start 132.8 103.3) (end 132.8 102.550678) (width 0.1) (layer "F.Cu") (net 2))
 (segment (start 136.799678 98.551) (end 141.728232 98.551) (width 0.1) (layer "F.Cu") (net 2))
 (via (at 141.614634 95.985366) (size 0.6) (drill 0.3) (layers "F.Cu" "B.Cu") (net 2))
 (segment (start 139.50025 96.5113) (end 139.50025 96.9923) (width 0.1) (layer "B.Cu") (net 2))
 (segment (start 141.614634 95.985366) (end 140.026184 95.985366) (width 0.1) (layer "B.Cu") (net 2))
 (segment (start 140.026184 95.985366) (end 139.50025 96.5113) (width 0.1) (layer "B.Cu") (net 2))
 (segment (start 135.386144 92.725366) (end 133.1 95.01151) (width 0.1) (layer "F.Cu") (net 12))
 (segment (start 145.061 94.821398) (end 142.964968 92.725366) (width 0.1) (layer "F.Cu") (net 12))
 (segment (start 138.806002 101.561) (end 142.975012 101.561) (width 0.1) (layer "F.Cu") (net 12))
 (segment (start 133.1 95.01151) (end 133.1 95.9) (width 0.1) (layer "F.Cu") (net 12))
 (segment (start 137.8 102.567002) (end 138.806002 101.561) (width 0.1) (layer "F.Cu") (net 12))
 (segment (start 142.975012 101.561) (end 145.061 99.475012) (width 0.1) (layer "F.Cu") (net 12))
 (segment (start 137.8 103.3) (end 137.8 102.567002) (width 0.1) (layer "F.Cu") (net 12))
 (segment (start 145.061 99.475012) (end 145.061 94.821398) (width 0.1) (layer "F.Cu") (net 12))
 (segment (start 142.964968 92.725366) (end 135.386144 92.725366) (width 0.1) (layer "F.Cu") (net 12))
 (via (at 133.1 95.9) (size 0.6) (drill 0.3) (layers "F.Cu" "B.Cu") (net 12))
 (segment (start 133.1 96.3) (end 133.15025 96.35025) (width 0.1) (layer "B.Cu") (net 12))
 (segment (start 133.1 95.9) (end 133.1 96.3) (width 0.1) (layer "B.Cu") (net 12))
 (segment (start 133.15025 96.35025) (end 133.15025 96.9923) (width 0.1) (layer "B.Cu") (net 12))
 (segment (start 132.3 99.60785) (end 133.15025 98.7576) (width 0.1) (layer "B.Cu") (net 14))
 (segment (start 132.3 103.3) (end 132.3 99.60785) (width 0.1) (layer "B.Cu") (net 14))
 (segment (start 133.15025 98.7576) (end 133.15025 97.9321) (width 0.1) (layer "B.Cu") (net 14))
 (segment (start 134.3 99.76085) (end 135.69025 98.3706) (width 0.1) (layer "B.Cu") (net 18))
 (segment (start 134.3 103.3) (end 134.3 99.76085) (width 0.1) (layer "B.Cu") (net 18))
 (segment (start 135.69025 98.3706) (end 135.69025 97.9321) (width 0.1) (layer "B.Cu") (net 18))
 (segment (start 142.653 98.477588) (end 142.653 95.818822) (width 0.1) (layer "F.Cu") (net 4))
 (segment (start 137.247 99.153) (end 141.977588 99.153) (width 0.1) (layer "F.Cu") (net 4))
 (segment (start 141.967544 95.133366) (end 139.029035 95.133366) (width 0.1) (layer "F.Cu") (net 4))
 (segment (start 133.8 103.3) (end 133.8 102.6) (width 0.1) (layer "F.Cu") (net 4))
 (segment (start 141.977588 99.153) (end 142.653 98.477588) (width 0.1) (layer "F.Cu") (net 4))
 (segment (start 133.8 102.6) (end 137.247 99.153) (width 0.1) (layer "F.Cu") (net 4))
 (segment (start 142.653 95.818822) (end 141.967544 95.133366) (width 0.1) (layer "F.Cu") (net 4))
 (segment (start 139.029035 95.133366) (end 138.589114 95.573287) (width 0.1) (layer "F.Cu") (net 4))
 (via (at 138.589114 95.573287) (size 0.6) (drill 0.3) (layers "F.Cu" "B.Cu") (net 4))
 (segment (start 138.589114 95.573287) (end 138.23025 95.932151) (width 0.1) (layer "B.Cu") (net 4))
 (segment (start 138.23025 95.932151) (end 138.23025 96.9923) (width 0.1) (layer "B.Cu") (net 4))
 (segment (start 136.925 98) (end 141.5 98) (width 0.1) (layer "F.Cu") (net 1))
 (segment (start 132.3 102.625) (end 136.925 98) (width 0.1) (layer "F.Cu") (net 1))
 (segment (start 132.3 103.3) (end 132.3 102.625) (width 0.1) (layer "F.Cu") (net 1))
 (via (at 141.5 98) (size 0.6) (drill 0.3) (layers "F.Cu" "B.Cu") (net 1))
 (segment (start 141.5 96.64855) (end 141.21175 96.3603) (width 0.1) (layer "B.Cu") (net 1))
 (segment (start 141.5 98) (end 141.5 96.64855) (width 0.1) (layer "B.Cu") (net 1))
 (segment (start 140.28625 96.3603) (end 140.13525 96.5113) (width 0.1) (layer "B.Cu") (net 1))
 (segment (start 140.13525 96.5113) (end 140.13525 96.9923) (width 0.1) (layer "B.Cu") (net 1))
 (segment (start 141.21175 96.3603) (end 140.28625 96.3603) (width 0.1) (layer "B.Cu") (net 1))
 (segment (start 142.351622 100.056) (end 143.556 98.851622) (width 0.1) (layer "F.Cu") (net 7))
 (segment (start 143.556 98.851622) (end 143.556 95.444788) (width 0.1) (layer "F.Cu") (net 7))
 (segment (start 137.844 100.056) (end 142.351622 100.056) (width 0.1) (layer "F.Cu") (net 7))
 (segment (start 136.304462 95.515211) (end 136.304462 95.597945) (width 0.1) (layer "F.Cu") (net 7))
 (segment (start 137.589307 94.230366) (end 136.304462 95.515211) (width 0.1) (layer "F.Cu") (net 7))
 (segment (start 135.3 103.3) (end 135.3 102.6) (width 0.1) (layer "F.Cu") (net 7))
 (segment (start 143.556 95.444788) (end 142.341578 94.230366) (width 0.1) (layer "F.Cu") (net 7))
 (segment (start 142.341578 94.230366) (end 137.589307 94.230366) (width 0.1) (layer "F.Cu") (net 7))
 (segment (start 135.3 102.6) (end 137.844 100.056) (width 0.1) (layer "F.Cu") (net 7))
 (via (at 136.304462 95.597945) (size 0.6) (drill 0.3) (layers "F.Cu" "B.Cu") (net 7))
 (segment (start 136.32525 95.618733) (end 136.32525 96.9923) (width 0.1) (layer "B.Cu") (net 7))
 (segment (start 136.304462 95.597945) (end 136.32525 95.618733) (width 0.1) (layer "B.Cu") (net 7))
 (segment (start 134.42025 98.338956) (end 134.42025 97.9321) (width 0.1) (layer "B.Cu") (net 16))
 (segment (start 133.3 99.459206) (end 134.42025 98.338956) (width 0.1) (layer "B.Cu") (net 16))
 (segment (start 133.3 103.3) (end 133.3 99.459206) (width 0.1) (layer "B.Cu") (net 16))
 (segment (start 134.8 103.3) (end 134.8 99.93835) (width 0.1) (layer "B.Cu") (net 19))
 (segment (start 136.32525 98.4131) (end 136.32525 97.9321) (width 0.1) (layer "B.Cu") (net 19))
 (segment (start 134.8 99.93835) (end 136.32525 98.4131) (width 0.1) (layer "B.Cu") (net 19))
 (segment (start 139.50025 98.3706) (end 139.50025 97.9321) (width 0.1) (layer "B.Cu") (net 24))
 (segment (start 137.3 103.3) (end 137.3 100.57085) (width 0.1) (layer "B.Cu") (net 24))
 (segment (start 137.3 100.57085) (end 139.50025 98.3706) (width 0.1) (layer "B.Cu") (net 24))
 (segment (start 137.8 103.3) (end 137.8 100.70585) (width 0.1) (layer "B.Cu") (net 25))
 (segment (start 137.8 100.70585) (end 140.13525 98.3706) (width 0.1) (layer "B.Cu") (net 25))
 (segment (start 140.13525 98.3706) (end 140.13525 97.9321) (width 0.1) (layer "B.Cu") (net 25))
 (segment (start 135.05525 98.3706) (end 135.05525 97.9321) (width 0.1) (layer "B.Cu") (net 17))
 (segment (start 133.8 103.3) (end 133.8 99.62585) (width 0.1) (layer "B.Cu") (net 17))
 (segment (start 133.8 99.62585) (end 135.05525 98.3706) (width 0.1) (layer "B.Cu") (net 17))
 (segment (start 136.8 100.43585) (end 138.86525 98.3706) (width 0.1) (layer "B.Cu") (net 23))
 (segment (start 138.86525 98.3706) (end 138.86525 97.9321) (width 0.1) (layer "B.Cu") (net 23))
 (segment (start 136.8 103.3) (end 136.8 100.43585) (width 0.1) (layer "B.Cu") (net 23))
 (segment (start 132.8 103.3) (end 132.8 99.533528) (width 0.1) (layer "B.Cu") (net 15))
 (segment (start 133.78525 98.548278) (end 133.78525 97.9321) (width 0.1) (layer "B.Cu") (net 15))
 (segment (start 132.8 99.533528) (end 133.78525 98.548278) (width 0.1) (layer "B.Cu") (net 15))
 (segment (start 135.3 100.03085) (end 136.96025 98.3706) (width 0.1) (layer "B.Cu") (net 20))
 (segment (start 136.96025 98.3706) (end 136.96025 97.9321) (width 0.1) (layer "B.Cu") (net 20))
 (segment (start 135.3 103.3) (end 135.3 100.03085) (width 0.1) (layer "B.Cu") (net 20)))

